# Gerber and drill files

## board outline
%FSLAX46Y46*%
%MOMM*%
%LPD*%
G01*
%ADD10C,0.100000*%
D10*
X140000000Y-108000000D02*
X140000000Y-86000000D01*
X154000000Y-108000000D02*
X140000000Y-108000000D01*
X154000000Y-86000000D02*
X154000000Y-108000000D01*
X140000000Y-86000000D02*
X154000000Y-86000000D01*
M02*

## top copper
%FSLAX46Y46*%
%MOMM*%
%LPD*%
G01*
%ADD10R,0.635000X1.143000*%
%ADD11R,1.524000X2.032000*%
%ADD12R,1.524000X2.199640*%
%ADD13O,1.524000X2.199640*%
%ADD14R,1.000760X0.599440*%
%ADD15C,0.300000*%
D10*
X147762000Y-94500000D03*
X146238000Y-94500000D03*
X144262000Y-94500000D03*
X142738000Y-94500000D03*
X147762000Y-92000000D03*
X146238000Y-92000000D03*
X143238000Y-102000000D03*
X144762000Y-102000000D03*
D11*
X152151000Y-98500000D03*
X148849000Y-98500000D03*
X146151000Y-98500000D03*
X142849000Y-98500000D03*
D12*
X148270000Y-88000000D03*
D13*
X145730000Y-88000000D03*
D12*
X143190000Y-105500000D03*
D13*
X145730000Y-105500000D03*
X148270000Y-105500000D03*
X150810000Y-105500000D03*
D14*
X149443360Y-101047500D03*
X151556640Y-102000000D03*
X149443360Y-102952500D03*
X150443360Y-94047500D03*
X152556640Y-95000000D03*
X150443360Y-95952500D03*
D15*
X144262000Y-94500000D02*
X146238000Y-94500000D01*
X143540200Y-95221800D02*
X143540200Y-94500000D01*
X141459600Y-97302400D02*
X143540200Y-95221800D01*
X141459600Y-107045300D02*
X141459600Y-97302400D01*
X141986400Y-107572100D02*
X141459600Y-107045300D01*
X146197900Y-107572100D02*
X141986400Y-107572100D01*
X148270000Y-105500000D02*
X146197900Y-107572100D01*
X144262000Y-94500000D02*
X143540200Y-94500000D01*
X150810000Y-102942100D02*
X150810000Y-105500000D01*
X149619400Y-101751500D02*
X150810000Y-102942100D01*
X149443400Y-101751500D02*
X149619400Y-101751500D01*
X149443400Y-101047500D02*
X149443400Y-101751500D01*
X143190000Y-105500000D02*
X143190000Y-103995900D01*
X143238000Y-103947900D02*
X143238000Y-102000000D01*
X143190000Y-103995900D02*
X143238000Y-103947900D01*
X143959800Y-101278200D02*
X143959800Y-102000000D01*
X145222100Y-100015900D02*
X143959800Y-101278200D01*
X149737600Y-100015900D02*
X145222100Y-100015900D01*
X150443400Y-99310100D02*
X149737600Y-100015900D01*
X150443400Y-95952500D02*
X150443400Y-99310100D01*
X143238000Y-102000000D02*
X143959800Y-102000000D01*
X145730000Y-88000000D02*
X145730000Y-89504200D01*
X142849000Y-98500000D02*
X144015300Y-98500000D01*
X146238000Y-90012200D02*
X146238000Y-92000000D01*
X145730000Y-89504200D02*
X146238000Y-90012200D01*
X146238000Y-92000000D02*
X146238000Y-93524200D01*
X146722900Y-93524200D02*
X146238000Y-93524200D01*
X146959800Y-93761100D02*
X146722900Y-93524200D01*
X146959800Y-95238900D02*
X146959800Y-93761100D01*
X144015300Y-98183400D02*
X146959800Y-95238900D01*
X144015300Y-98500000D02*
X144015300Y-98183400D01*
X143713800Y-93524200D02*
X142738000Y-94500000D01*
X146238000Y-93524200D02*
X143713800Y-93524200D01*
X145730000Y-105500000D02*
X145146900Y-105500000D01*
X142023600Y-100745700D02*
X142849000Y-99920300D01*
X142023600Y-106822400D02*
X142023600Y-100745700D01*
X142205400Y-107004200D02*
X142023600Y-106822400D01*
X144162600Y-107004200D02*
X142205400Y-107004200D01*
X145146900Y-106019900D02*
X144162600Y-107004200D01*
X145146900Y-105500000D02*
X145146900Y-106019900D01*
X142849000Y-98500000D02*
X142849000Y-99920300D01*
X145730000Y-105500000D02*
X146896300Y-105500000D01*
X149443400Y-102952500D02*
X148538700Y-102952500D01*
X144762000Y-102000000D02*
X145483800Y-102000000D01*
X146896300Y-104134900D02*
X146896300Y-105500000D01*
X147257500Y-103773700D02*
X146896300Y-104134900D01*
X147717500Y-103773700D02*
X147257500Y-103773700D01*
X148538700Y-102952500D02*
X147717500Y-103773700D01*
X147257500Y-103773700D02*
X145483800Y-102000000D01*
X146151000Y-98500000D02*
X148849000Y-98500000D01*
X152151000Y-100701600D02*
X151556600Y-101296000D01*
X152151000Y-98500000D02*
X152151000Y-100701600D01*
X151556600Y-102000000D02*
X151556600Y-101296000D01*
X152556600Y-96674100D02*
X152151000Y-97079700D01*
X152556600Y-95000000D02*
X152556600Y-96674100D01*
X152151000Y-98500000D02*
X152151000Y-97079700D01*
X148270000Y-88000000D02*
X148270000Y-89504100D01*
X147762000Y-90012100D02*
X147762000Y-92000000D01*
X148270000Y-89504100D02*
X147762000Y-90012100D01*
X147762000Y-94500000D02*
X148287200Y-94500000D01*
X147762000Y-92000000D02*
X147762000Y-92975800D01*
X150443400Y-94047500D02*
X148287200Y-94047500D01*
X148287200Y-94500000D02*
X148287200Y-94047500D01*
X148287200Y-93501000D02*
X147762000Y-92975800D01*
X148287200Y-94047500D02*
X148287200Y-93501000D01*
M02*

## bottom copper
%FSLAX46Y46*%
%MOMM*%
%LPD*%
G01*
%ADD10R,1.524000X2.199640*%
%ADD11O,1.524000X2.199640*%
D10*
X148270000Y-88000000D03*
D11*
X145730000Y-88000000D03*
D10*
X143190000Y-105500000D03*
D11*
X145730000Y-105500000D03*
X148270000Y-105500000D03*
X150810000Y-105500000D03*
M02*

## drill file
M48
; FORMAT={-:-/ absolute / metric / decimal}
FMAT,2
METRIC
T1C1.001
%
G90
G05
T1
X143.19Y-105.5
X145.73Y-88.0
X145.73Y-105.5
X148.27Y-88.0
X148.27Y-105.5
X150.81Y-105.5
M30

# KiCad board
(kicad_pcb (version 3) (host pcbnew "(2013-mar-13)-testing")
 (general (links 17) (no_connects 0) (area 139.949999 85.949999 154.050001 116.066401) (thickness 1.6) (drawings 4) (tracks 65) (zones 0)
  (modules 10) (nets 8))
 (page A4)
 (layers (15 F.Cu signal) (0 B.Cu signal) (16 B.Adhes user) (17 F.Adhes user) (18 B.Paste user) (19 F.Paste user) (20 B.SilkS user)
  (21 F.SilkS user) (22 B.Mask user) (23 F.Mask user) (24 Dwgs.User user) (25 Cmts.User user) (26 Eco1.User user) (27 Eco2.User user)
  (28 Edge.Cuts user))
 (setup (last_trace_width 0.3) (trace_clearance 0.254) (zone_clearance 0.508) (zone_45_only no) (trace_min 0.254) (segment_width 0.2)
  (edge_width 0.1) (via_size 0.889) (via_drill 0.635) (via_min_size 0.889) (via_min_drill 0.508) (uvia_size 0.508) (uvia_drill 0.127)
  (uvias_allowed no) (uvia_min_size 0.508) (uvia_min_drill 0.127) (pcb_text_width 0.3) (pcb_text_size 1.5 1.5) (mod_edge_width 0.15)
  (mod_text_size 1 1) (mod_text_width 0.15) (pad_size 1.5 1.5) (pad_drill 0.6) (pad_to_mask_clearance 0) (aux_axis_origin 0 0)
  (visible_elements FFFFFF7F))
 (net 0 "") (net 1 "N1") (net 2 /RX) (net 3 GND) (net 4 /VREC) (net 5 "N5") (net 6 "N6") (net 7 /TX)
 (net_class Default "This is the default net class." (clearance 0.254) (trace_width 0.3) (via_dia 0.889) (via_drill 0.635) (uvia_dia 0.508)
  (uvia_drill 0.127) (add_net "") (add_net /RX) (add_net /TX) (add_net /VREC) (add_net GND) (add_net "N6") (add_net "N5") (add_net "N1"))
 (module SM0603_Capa (layer F.Cu) (at 147 94.5 180)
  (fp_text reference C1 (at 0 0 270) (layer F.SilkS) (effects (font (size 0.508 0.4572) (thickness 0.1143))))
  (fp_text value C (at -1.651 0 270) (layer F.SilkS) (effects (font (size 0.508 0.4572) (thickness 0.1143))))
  (pad 1 smd rect (at -0.762 0 180) (size 0.635 1.143) (layers F.Cu F.Paste F.Mask) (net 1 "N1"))
  (pad 2 smd rect (at 0.762 0 180) (size 0.635 1.143) (layers F.Cu F.Paste F.Mask) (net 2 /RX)))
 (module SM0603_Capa (layer F.Cu) (at 143.5 94.5 180)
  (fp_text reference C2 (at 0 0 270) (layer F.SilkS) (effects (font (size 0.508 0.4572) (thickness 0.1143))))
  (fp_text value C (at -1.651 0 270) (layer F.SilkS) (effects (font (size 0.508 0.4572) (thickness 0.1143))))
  (pad 1 smd rect (at -0.762 0 180) (size 0.635 1.143) (layers F.Cu F.Paste F.Mask) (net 2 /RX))
  (pad 2 smd rect (at 0.762 0 180) (size 0.635 1.143) (layers F.Cu F.Paste F.Mask) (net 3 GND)))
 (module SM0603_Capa (layer F.Cu) (at 147 92 180)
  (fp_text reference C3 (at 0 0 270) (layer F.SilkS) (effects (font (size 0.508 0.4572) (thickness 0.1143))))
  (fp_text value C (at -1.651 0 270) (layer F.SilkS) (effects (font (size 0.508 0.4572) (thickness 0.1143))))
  (pad 1 smd rect (at -0.762 0 180) (size 0.635 1.143) (layers F.Cu F.Paste F.Mask) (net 1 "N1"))
  (pad 2 smd rect (at 0.762 0 180) (size 0.635 1.143) (layers F.Cu F.Paste F.Mask) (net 3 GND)))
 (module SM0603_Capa (layer F.Cu) (at 144 102)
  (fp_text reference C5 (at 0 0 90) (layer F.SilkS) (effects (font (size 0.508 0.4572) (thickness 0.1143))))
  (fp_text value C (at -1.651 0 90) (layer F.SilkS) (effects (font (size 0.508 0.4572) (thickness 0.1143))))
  (pad 1 smd rect (at -0.762 0) (size 0.635 1.143) (layers F.Cu F.Paste F.Mask) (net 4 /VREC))
  (pad 2 smd rect (at 0.762 0) (size 0.635 1.143) (layers F.Cu F.Paste F.Mask) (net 3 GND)))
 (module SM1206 (layer F.Cu) (at 150.5 98.5 180)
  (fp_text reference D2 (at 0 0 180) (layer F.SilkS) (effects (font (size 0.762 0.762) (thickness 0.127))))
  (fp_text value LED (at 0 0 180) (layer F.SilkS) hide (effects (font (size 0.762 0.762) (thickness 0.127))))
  (pad 1 smd rect (at -1.651 0 180) (size 1.524 2.032) (layers F.Cu F.Paste F.Mask) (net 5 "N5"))
  (pad 2 smd rect (at 1.651 0 180) (size 1.524 2.032) (layers F.Cu F.Paste F.Mask) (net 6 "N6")))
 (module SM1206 (layer F.Cu) (at 144.5 98.5 180)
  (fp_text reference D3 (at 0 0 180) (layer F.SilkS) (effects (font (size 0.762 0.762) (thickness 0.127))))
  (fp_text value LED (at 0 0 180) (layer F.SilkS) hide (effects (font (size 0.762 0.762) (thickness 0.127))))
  (pad 1 smd rect (at -1.651 0 180) (size 1.524 2.032) (layers F.Cu F.Paste F.Mask) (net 6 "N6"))
  (pad 2 smd rect (at 1.651 0 180) (size 1.524 2.032) (layers F.Cu F.Paste F.Mask) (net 3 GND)))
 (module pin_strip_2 (layer F.Cu) (at 147 88 180)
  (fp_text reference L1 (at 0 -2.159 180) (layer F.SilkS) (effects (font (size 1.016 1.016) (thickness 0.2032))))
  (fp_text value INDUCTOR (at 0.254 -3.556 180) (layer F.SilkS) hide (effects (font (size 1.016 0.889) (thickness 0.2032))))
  (pad 1 thru_hole rect (at -1.27 0 180) (size 1.524 2.19964) (drill 1.00076) (layers *.Cu *.Mask F.SilkS) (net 1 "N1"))
  (pad 2 thru_hole oval (at 1.27 0 180) (size 1.524 2.19964) (drill 1.00076) (layers *.Cu *.Mask F.SilkS) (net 3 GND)))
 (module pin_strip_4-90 (layer F.Cu) (at 147 105.5)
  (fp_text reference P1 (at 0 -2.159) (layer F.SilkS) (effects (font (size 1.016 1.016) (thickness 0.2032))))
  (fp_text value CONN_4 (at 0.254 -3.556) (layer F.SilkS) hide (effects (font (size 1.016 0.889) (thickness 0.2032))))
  (pad 1 thru_hole rect (at -3.81 0) (size 1.524 2.19964) (drill 1.00076) (layers *.Cu *.Mask F.SilkS) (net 4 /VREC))
  (pad 2 thru_hole oval (at -1.27 0) (size 1.524 2.19964) (drill 1.00076) (layers *.Cu *.Mask F.SilkS) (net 3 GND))
  (pad 3 thru_hole oval (at 1.27 0) (size 1.524 2.19964) (drill 1.00076) (layers *.Cu *.Mask F.SilkS) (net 2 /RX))
  (pad 4 thru_hole oval (at 3.81 0) (size 1.524 2.19964) (drill 1.00076) (layers *.Cu *.Mask F.SilkS) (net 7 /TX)))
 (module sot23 (layer F.Cu) (at 150.5 102 270)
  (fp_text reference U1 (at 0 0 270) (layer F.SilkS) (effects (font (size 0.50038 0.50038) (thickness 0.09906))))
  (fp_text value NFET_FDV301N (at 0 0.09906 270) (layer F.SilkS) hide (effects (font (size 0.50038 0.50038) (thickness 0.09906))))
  (pad 1 smd rect (at -0.9525 1.05664 270) (size 0.59944 1.00076) (layers F.Cu F.Paste F.Mask) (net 7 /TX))
  (pad 2 smd rect (at 0 -1.05664 270) (size 0.59944 1.00076) (layers F.Cu F.Paste F.Mask) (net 5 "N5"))
  (pad 3 smd rect (at 0.9525 1.05664 270) (size 0.59944 1.00076) (layers F.Cu F.Paste F.Mask) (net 3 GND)))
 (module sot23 (layer F.Cu) (at 151.5 95 270)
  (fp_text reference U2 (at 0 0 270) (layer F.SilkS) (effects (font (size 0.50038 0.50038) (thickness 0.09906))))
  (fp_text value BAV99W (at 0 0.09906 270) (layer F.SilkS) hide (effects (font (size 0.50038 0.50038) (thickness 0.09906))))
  (pad 1 smd rect (at -0.9525 1.05664 270) (size 0.59944 1.00076) (layers F.Cu F.Paste F.Mask) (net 1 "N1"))
  (pad 2 smd rect (at 0 -1.05664 270) (size 0.59944 1.00076) (layers F.Cu F.Paste F.Mask) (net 5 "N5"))
  (pad 3 smd rect (at 0.9525 1.05664 270) (size 0.59944 1.00076) (layers F.Cu F.Paste F.Mask) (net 4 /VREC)))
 (gr_line (start 140 108) (end 140 86) (angle 90) (layer Edge.Cuts) (width 0.1))
 (gr_line (start 154 108) (end 140 108) (angle 90) (layer Edge.Cuts) (width 0.1))
 (gr_line (start 154 86) (end 154 108) (angle 90) (layer Edge.Cuts) (width 0.1))
 (gr_line (start 140 86) (end 154 86) (angle 90) (layer Edge.Cuts) (width 0.1))
 (segment (start 144.262 94.5) (end 146.238 94.5) (width 0.3) (layer F.Cu) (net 2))
 (segment (start 143.5402 95.2218) (end 143.5402 94.5) (width 0.3) (layer F.Cu) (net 2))
 (segment (start 141.4596 97.3024) (end 143.5402 95.2218) (width 0.3) (layer F.Cu) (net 2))
 (segment (start 141.4596 107.0453) (end 141.4596 97.3024) (width 0.3) (layer F.Cu) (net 2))
 (segment (start 141.9864 107.5721) (end 141.4596 107.0453) (width 0.3) (layer F.Cu) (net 2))
 (segment (start 146.1979 107.5721) (end 141.9864 107.5721) (width 0.3) (layer F.Cu) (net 2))
 (segment (start 148.27 105.5) (end 146.1979 107.5721) (width 0.3) (layer F.Cu) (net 2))
 (segment (start 144.262 94.5) (end 143.5402 94.5) (width 0.3) (layer F.Cu) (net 2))
 (segment (start 150.81 102.9421) (end 150.81 105.5) (width 0.3) (layer F.Cu) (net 7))
 (segment (start 149.6194 101.7515) (end 150.81 102.9421) (width 0.3) (layer F.Cu) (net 7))
 (segment (start 149.4434 101.7515) (end 149.6194 101.7515) (width 0.3) (layer F.Cu) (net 7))
 (segment (start 149.4434 101.0475) (end 149.4434 101.7515) (width 0.3) (layer F.Cu) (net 7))
 (segment (start 143.19 105.5) (end 143.19 103.9959) (width 0.3) (layer F.Cu) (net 4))
 (segment (start 143.238 103.9479) (end 143.238 102) (width 0.3) (layer F.Cu) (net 4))
 (segment (start 143.19 103.9959) (end 143.238 103.9479) (width 0.3) (layer F.Cu) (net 4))
 (segment (start 143.9598 101.2782) (end 143.9598 102) (width 0.3) (layer F.Cu) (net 4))
 (segment (start 145.2221 100.0159) (end 143.9598 101.2782) (width 0.3) (layer F.Cu) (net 4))
 (segment (start 149.7376 100.0159) (end 145.2221 100.0159) (width 0.3) (layer F.Cu) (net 4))
 (segment (start 150.4434 99.3101) (end 149.7376 100.0159) (width 0.3) (layer F.Cu) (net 4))
 (segment (start 150.4434 95.9525) (end 150.4434 99.3101) (width 0.3) (layer F.Cu) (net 4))
 (segment (start 143.238 102) (end 143.9598 102) (width 0.3) (layer F.Cu) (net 4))
 (segment (start 145.73 88) (end 145.73 89.5042) (width 0.3) (layer F.Cu) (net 3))
 (segment (start 142.849 98.5) (end 144.0153 98.5) (width 0.3) (layer F.Cu) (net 3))
 (segment (start 146.238 90.0122) (end 146.238 92) (width 0.3) (layer F.Cu) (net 3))
 (segment (start 145.73 89.5042) (end 146.238 90.0122) (width 0.3) (layer F.Cu) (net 3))
 (segment (start 146.238 92) (end 146.238 93.5242) (width 0.3) (layer F.Cu) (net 3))
 (segment (start 146.7229 93.5242) (end 146.238 93.5242) (width 0.3) (layer F.Cu) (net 3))
 (segment (start 146.9598 93.7611) (end 146.7229 93.5242) (width 0.3) (layer F.Cu) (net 3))
 (segment (start 146.9598 95.2389) (end 146.9598 93.7611) (width 0.3) (layer F.Cu) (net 3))
 (segment (start 144.0153 98.1834) (end 146.9598 95.2389) (width 0.3) (layer F.Cu) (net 3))
 (segment (start 144.0153 98.5) (end 144.0153 98.1834) (width 0.3) (layer F.Cu) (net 3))
 (segment (start 143.7138 93.5242) (end 142.738 94.5) (width 0.3) (layer F.Cu) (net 3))
 (segment (start 146.238 93.5242) (end 143.7138 93.5242) (width 0.3) (layer F.Cu) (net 3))
 (segment (start 145.73 105.5) (end 145.1469 105.5) (width 0.3) (layer F.Cu) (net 3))
 (segment (start 142.0236 100.7457) (end 142.849 99.9203) (width 0.3) (layer F.Cu) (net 3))
 (segment (start 142.0236 106.8224) (end 142.0236 100.7457) (width 0.3) (layer F.Cu) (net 3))
 (segment (start 142.2054 107.0042) (end 142.0236 106.8224) (width 0.3) (layer F.Cu) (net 3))
 (segment (start 144.1626 107.0042) (end 142.2054 107.0042) (width 0.3) (layer F.Cu) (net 3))
 (segment (start 145.1469 106.0199) (end 144.1626 107.0042) (width 0.3) (layer F.Cu) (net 3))
 (segment (start 145.1469 105.5) (end 145.1469 106.0199) (width 0.3) (layer F.Cu) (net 3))
 (segment (start 142.849 98.5) (end 142.849 99.9203) (width 0.3) (layer F.Cu) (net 3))
 (segment (start 145.73 105.5) (end 146.8963 105.5) (width 0.3) (layer F.Cu) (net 3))
 (segment (start 149.4434 102.9525) (end 148.5387 102.9525) (width 0.3) (layer F.Cu) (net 3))
 (segment (start 144.762 102) (end 145.4838 102) (width 0.3) (layer F.Cu) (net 3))
 (segment (start 146.8963 104.1349) (end 146.8963 105.5) (width 0.3) (layer F.Cu) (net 3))
 (segment (start 147.2575 103.7737) (end 146.8963 104.1349) (width 0.3) (layer F.Cu) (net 3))
 (segment (start 147.7175 103.7737) (end 147.2575 103.7737) (width 0.3) (layer F.Cu) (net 3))
 (segment (start 148.5387 102.9525) (end 147.7175 103.7737) (width 0.3) (layer F.Cu) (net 3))
 (segment (start 147.2575 103.7737) (end 145.4838 102) (width 0.3) (layer F.Cu) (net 3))
 (segment (start 146.151 98.5) (end 148.849 98.5) (width 0.3) (layer F.Cu) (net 6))
 (segment (start 152.151 100.7016) (end 151.5566 101.296) (width 0.3) (layer F.Cu) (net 5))
 (segment (start 152.151 98.5) (end 152.151 100.7016) (width 0.3) (layer F.Cu) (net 5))
 (segment (start 151.5566 102) (end 151.5566 101.296) (width 0.3) (layer F.Cu) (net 5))
 (segment (start 152.5566 96.6741) (end 152.151 97.0797) (width 0.3) (layer F.Cu) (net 5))
 (segment (start 152.5566 95) (end 152.5566 96.6741) (width 0.3) (layer F.Cu) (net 5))
 (segment (start 152.151 98.5) (end 152.151 97.0797) (width 0.3) (layer F.Cu) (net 5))
 (segment (start 148.27 88) (end 148.27 89.5041) (width 0.3) (layer F.Cu) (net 1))
 (segment (start 147.762 90.0121) (end 147.762 92) (width 0.3) (layer F.Cu) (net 1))
 (segment (start 148.27 89.5041) (end 147.762 90.0121) (width 0.3) (layer F.Cu) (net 1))
 (segment (start 147.762 94.5) (end 148.2872 94.5) (width 0.3) (layer F.Cu) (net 1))
 (segment (start 147.762 92) (end 147.762 92.9758) (width 0.3) (layer F.Cu) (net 1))
 (segment (start 150.4434 94.0475) (end 148.2872 94.0475) (width 0.3) (layer F.Cu) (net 1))
 (segment (start 148.2872 94.5) (end 148.2872 94.0475) (width 0.3) (layer F.Cu) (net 1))
 (segment (start 148.2872 93.501) (end 147.762 92.9758) (width 0.3) (layer F.Cu) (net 1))
 (segment (start 148.2872 94.0475) (end 148.2872 93.501) (width 0.3) (layer F.Cu) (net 1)))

